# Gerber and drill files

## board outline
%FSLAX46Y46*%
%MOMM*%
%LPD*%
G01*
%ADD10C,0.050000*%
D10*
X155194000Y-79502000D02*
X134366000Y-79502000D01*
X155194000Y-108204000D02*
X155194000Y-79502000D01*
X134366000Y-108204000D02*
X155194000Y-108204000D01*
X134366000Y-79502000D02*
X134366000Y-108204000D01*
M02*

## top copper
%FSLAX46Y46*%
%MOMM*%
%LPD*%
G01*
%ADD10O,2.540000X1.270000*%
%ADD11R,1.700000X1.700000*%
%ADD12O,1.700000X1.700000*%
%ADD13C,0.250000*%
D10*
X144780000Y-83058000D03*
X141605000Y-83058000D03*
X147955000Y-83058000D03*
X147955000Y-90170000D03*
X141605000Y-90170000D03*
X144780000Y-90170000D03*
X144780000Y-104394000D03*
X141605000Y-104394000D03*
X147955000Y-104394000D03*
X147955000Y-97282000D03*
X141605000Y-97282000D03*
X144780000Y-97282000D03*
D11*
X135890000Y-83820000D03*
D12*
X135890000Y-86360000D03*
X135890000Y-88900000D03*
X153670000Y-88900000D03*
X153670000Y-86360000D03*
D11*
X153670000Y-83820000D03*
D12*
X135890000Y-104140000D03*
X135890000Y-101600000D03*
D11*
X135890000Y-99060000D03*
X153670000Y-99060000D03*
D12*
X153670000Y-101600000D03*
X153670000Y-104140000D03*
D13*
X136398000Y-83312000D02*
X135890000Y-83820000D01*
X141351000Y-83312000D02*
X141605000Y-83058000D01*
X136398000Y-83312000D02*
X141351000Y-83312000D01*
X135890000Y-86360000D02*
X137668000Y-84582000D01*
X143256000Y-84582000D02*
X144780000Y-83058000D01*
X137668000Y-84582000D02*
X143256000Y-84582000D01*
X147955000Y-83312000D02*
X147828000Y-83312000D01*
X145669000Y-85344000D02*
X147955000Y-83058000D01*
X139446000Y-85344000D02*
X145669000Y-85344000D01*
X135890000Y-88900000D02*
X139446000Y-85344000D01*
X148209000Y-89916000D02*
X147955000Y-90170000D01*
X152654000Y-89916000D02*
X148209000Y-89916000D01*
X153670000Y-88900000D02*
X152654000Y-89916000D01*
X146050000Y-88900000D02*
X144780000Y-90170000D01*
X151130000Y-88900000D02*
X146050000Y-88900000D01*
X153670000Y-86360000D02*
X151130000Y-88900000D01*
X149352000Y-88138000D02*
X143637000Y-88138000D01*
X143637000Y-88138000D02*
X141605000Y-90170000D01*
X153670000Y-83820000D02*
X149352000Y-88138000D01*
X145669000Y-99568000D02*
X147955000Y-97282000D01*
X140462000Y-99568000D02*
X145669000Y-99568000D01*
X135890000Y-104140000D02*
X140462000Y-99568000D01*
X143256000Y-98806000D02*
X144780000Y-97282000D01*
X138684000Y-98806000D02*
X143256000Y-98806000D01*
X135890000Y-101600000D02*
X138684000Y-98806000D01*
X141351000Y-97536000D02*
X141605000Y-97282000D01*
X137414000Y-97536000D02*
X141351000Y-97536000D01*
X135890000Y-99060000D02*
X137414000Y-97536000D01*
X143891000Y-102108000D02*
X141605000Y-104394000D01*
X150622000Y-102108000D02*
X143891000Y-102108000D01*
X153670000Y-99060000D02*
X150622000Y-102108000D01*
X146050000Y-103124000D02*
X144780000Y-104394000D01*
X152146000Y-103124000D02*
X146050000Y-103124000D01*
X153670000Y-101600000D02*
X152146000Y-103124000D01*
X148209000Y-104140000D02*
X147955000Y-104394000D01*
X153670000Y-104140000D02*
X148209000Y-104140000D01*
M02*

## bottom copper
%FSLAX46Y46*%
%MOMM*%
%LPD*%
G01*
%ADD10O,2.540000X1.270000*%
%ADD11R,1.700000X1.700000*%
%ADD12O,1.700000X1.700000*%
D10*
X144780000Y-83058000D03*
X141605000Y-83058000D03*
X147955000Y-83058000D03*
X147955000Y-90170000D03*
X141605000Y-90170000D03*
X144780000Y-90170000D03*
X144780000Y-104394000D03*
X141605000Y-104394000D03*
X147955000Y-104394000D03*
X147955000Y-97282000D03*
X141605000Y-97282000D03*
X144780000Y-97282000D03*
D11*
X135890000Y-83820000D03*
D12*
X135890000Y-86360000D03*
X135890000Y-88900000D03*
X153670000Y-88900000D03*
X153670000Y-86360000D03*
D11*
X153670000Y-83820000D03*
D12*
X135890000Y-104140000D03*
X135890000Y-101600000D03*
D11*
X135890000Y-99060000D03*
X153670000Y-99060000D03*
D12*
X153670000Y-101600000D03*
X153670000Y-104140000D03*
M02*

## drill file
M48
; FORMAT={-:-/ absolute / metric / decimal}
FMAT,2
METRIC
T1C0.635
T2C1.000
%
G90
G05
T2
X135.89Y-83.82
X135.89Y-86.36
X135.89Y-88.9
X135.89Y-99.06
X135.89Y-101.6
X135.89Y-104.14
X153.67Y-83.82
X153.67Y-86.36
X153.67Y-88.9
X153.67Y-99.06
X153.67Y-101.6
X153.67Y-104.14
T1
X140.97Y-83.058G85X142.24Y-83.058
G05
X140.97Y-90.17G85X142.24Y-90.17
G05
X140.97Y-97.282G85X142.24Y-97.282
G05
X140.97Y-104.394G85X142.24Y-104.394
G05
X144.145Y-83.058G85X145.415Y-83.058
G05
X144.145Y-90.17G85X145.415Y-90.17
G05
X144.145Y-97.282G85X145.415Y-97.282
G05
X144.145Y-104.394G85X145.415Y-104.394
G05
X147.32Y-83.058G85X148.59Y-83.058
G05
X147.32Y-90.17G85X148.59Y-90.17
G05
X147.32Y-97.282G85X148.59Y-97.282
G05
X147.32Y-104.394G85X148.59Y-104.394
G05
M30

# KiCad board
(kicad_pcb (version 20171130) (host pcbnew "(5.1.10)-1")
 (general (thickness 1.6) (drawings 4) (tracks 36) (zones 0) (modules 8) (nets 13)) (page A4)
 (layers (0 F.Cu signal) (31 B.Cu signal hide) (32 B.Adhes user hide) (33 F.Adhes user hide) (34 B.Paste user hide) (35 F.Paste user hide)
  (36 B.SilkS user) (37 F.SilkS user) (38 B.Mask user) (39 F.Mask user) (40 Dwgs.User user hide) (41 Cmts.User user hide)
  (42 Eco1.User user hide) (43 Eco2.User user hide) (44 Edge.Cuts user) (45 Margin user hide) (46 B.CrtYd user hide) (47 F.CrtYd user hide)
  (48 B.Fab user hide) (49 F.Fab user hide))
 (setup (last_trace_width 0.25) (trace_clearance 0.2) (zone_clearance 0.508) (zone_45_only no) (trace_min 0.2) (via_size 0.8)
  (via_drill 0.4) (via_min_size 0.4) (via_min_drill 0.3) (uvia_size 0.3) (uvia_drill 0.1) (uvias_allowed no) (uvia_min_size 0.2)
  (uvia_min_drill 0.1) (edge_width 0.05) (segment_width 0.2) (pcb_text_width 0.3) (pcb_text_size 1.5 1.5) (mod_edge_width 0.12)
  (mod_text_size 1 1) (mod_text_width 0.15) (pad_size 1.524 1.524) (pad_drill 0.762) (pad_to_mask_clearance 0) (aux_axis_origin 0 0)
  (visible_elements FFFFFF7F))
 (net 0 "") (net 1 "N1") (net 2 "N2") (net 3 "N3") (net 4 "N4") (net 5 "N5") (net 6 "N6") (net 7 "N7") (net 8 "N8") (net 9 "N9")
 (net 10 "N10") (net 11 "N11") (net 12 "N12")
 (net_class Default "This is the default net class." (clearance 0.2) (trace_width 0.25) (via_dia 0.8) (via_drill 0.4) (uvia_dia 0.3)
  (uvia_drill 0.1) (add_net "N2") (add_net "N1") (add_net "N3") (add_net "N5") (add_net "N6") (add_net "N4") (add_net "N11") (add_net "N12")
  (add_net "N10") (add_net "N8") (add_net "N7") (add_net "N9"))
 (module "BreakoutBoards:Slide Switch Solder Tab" (layer F.Cu) (at 144.78 83.058 90)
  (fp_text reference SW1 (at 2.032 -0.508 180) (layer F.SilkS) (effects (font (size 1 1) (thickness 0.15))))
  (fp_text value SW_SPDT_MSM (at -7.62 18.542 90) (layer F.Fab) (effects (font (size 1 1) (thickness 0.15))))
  (pad 2 thru_hole oval (at 0 0 90) (size 1.27 2.54) (drill oval 0.635 1.905) (layers *.Cu *.Mask) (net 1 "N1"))
  (pad 1 thru_hole oval (at 0 -3.175 90) (size 1.27 2.54) (drill oval 0.635 1.905) (layers *.Cu *.Mask) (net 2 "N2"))
  (pad 3 thru_hole oval (at 0 3.175 90) (size 1.27 2.54) (drill oval 0.635 1.905) (layers *.Cu *.Mask) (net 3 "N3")))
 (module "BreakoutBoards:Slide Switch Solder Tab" (layer F.Cu) (at 144.78 90.17 90)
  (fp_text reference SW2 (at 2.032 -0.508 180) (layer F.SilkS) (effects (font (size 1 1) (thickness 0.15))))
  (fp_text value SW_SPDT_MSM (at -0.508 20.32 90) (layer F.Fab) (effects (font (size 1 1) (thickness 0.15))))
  (pad 3 thru_hole oval (at 0 3.175 90) (size 1.27 2.54) (drill oval 0.635 1.905) (layers *.Cu *.Mask) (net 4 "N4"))
  (pad 1 thru_hole oval (at 0 -3.175 90) (size 1.27 2.54) (drill oval 0.635 1.905) (layers *.Cu *.Mask) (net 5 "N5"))
  (pad 2 thru_hole oval (at 0 0 90) (size 1.27 2.54) (drill oval 0.635 1.905) (layers *.Cu *.Mask) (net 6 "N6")))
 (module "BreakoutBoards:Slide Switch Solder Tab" (layer F.Cu) (at 144.78 104.394 90)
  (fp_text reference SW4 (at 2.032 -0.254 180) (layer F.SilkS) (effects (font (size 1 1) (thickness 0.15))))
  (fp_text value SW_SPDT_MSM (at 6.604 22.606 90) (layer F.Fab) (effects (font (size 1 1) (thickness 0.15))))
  (pad 2 thru_hole oval (at 0 0 90) (size 1.27 2.54) (drill oval 0.635 1.905) (layers *.Cu *.Mask) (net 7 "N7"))
  (pad 1 thru_hole oval (at 0 -3.175 90) (size 1.27 2.54) (drill oval 0.635 1.905) (layers *.Cu *.Mask) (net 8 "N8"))
  (pad 3 thru_hole oval (at 0 3.175 90) (size 1.27 2.54) (drill oval 0.635 1.905) (layers *.Cu *.Mask) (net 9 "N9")))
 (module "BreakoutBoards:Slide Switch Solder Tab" (layer F.Cu) (at 144.78 97.282 90)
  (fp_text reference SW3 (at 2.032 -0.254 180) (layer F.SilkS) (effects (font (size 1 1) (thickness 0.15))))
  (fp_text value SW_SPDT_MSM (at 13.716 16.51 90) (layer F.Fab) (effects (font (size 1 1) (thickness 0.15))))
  (pad 3 thru_hole oval (at 0 3.175 90) (size 1.27 2.54) (drill oval 0.635 1.905) (layers *.Cu *.Mask) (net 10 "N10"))
  (pad 1 thru_hole oval (at 0 -3.175 90) (size 1.27 2.54) (drill oval 0.635 1.905) (layers *.Cu *.Mask) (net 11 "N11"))
  (pad 2 thru_hole oval (at 0 0 90) (size 1.27 2.54) (drill oval 0.635 1.905) (layers *.Cu *.Mask) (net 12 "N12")))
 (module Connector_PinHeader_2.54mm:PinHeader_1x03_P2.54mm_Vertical (layer F.Cu) (at 135.89 83.82)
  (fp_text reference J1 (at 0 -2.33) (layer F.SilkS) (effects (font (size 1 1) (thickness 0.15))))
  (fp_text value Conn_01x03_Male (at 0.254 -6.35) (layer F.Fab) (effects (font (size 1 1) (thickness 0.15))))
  (pad 1 thru_hole rect (at 0 0) (size 1.7 1.7) (drill 1) (layers *.Cu *.Mask) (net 2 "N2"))
  (pad 2 thru_hole oval (at 0 2.54) (size 1.7 1.7) (drill 1) (layers *.Cu *.Mask) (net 1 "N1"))
  (pad 3 thru_hole oval (at 0 5.08) (size 1.7 1.7) (drill 1) (layers *.Cu *.Mask) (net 3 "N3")))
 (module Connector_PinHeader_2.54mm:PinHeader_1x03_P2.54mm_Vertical (layer F.Cu) (at 153.67 83.82)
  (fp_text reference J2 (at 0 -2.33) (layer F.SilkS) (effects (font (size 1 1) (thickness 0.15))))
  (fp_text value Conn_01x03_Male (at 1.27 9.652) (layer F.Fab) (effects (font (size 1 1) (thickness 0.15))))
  (pad 3 thru_hole oval (at 0 5.08) (size 1.7 1.7) (drill 1) (layers *.Cu *.Mask) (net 4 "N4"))
  (pad 2 thru_hole oval (at 0 2.54) (size 1.7 1.7) (drill 1) (layers *.Cu *.Mask) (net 6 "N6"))
  (pad 1 thru_hole rect (at 0 0) (size 1.7 1.7) (drill 1) (layers *.Cu *.Mask) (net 5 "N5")))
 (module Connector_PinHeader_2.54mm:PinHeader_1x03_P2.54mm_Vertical (layer F.Cu) (at 135.89 99.06)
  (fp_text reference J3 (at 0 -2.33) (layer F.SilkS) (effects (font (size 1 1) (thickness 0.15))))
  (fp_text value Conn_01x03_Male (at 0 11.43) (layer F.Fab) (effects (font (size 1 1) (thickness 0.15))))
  (pad 3 thru_hole oval (at 0 5.08) (size 1.7 1.7) (drill 1) (layers *.Cu *.Mask) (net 10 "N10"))
  (pad 2 thru_hole oval (at 0 2.54) (size 1.7 1.7) (drill 1) (layers *.Cu *.Mask) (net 12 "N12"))
  (pad 1 thru_hole rect (at 0 0) (size 1.7 1.7) (drill 1) (layers *.Cu *.Mask) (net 11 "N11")))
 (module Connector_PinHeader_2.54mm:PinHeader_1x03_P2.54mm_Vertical (layer F.Cu) (at 153.67 99.06)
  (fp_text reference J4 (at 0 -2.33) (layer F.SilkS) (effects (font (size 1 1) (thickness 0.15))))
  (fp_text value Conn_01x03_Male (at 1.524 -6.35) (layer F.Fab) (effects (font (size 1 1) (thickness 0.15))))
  (pad 1 thru_hole rect (at 0 0) (size 1.7 1.7) (drill 1) (layers *.Cu *.Mask) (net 8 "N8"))
  (pad 2 thru_hole oval (at 0 2.54) (size 1.7 1.7) (drill 1) (layers *.Cu *.Mask) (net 7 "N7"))
  (pad 3 thru_hole oval (at 0 5.08) (size 1.7 1.7) (drill 1) (layers *.Cu *.Mask) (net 9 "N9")))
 (gr_line (start 155.194 79.502) (end 134.366 79.502) (layer Edge.Cuts) (width 0.05))
 (gr_line (start 155.194 108.204) (end 155.194 79.502) (layer Edge.Cuts) (width 0.05))
 (gr_line (start 134.366 108.204) (end 155.194 108.204) (layer Edge.Cuts) (width 0.05))
 (gr_line (start 134.366 79.502) (end 134.366 108.204) (layer Edge.Cuts) (width 0.05))
 (segment (start 136.398 83.312) (end 135.89 83.82) (width 0.25) (layer F.Cu) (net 2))
 (segment (start 141.351 83.312) (end 141.605 83.058) (width 0.25) (layer F.Cu) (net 2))
 (segment (start 136.398 83.312) (end 141.351 83.312) (width 0.25) (layer F.Cu) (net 2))
 (segment (start 135.89 86.36) (end 137.668 84.582) (width 0.25) (layer F.Cu) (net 1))
 (segment (start 143.256 84.582) (end 144.78 83.058) (width 0.25) (layer F.Cu) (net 1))
 (segment (start 137.668 84.582) (end 143.256 84.582) (width 0.25) (layer F.Cu) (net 1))
 (segment (start 147.955 83.312) (end 147.828 83.312) (width 0.25) (layer F.Cu) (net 3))
 (segment (start 145.669 85.344) (end 147.955 83.058) (width 0.25) (layer F.Cu) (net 3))
 (segment (start 139.446 85.344) (end 145.669 85.344) (width 0.25) (layer F.Cu) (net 3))
 (segment (start 135.89 88.9) (end 139.446 85.344) (width 0.25) (layer F.Cu) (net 3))
 (segment (start 148.209 89.916) (end 147.955 90.17) (width 0.25) (layer F.Cu) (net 4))
 (segment (start 152.654 89.916) (end 148.209 89.916) (width 0.25) (layer F.Cu) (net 4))
 (segment (start 153.67 88.9) (end 152.654 89.916) (width 0.25) (layer F.Cu) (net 4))
 (segment (start 146.05 88.9) (end 144.78 90.17) (width 0.25) (layer F.Cu) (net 6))
 (segment (start 151.13 88.9) (end 146.05 88.9) (width 0.25) (layer F.Cu) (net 6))
 (segment (start 153.67 86.36) (end 151.13 88.9) (width 0.25) (layer F.Cu) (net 6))
 (segment (start 149.352 88.138) (end 143.637 88.138) (width 0.25) (layer F.Cu) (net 5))
 (segment (start 143.637 88.138) (end 141.605 90.17) (width 0.25) (layer F.Cu) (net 5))
 (segment (start 153.67 83.82) (end 149.352 88.138) (width 0.25) (layer F.Cu) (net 5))
 (segment (start 145.669 99.568) (end 147.955 97.282) (width 0.25) (layer F.Cu) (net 10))
 (segment (start 140.462 99.568) (end 145.669 99.568) (width 0.25) (layer F.Cu) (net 10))
 (segment (start 135.89 104.14) (end 140.462 99.568) (width 0.25) (layer F.Cu) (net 10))
 (segment (start 143.256 98.806) (end 144.78 97.282) (width 0.25) (layer F.Cu) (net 12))
 (segment (start 138.684 98.806) (end 143.256 98.806) (width 0.25) (layer F.Cu) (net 12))
 (segment (start 135.89 101.6) (end 138.684 98.806) (width 0.25) (layer F.Cu) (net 12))
 (segment (start 141.351 97.536) (end 141.605 97.282) (width 0.25) (layer F.Cu) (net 11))
 (segment (start 137.414 97.536) (end 141.351 97.536) (width 0.25) (layer F.Cu) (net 11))
 (segment (start 135.89 99.06) (end 137.414 97.536) (width 0.25) (layer F.Cu) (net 11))
 (segment (start 143.891 102.108) (end 141.605 104.394) (width 0.25) (layer F.Cu) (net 8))
 (segment (start 150.622 102.108) (end 143.891 102.108) (width 0.25) (layer F.Cu) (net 8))
 (segment (start 153.67 99.06) (end 150.622 102.108) (width 0.25) (layer F.Cu) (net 8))
 (segment (start 146.05 103.124) (end 144.78 104.394) (width 0.25) (layer F.Cu) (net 7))
 (segment (start 152.146 103.124) (end 146.05 103.124) (width 0.25) (layer F.Cu) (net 7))
 (segment (start 153.67 101.6) (end 152.146 103.124) (width 0.25) (layer F.Cu) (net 7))
 (segment (start 148.209 104.14) (end 147.955 104.394) (width 0.25) (layer F.Cu) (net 9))
 (segment (start 153.67 104.14) (end 148.209 104.14) (width 0.25) (layer F.Cu) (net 9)))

